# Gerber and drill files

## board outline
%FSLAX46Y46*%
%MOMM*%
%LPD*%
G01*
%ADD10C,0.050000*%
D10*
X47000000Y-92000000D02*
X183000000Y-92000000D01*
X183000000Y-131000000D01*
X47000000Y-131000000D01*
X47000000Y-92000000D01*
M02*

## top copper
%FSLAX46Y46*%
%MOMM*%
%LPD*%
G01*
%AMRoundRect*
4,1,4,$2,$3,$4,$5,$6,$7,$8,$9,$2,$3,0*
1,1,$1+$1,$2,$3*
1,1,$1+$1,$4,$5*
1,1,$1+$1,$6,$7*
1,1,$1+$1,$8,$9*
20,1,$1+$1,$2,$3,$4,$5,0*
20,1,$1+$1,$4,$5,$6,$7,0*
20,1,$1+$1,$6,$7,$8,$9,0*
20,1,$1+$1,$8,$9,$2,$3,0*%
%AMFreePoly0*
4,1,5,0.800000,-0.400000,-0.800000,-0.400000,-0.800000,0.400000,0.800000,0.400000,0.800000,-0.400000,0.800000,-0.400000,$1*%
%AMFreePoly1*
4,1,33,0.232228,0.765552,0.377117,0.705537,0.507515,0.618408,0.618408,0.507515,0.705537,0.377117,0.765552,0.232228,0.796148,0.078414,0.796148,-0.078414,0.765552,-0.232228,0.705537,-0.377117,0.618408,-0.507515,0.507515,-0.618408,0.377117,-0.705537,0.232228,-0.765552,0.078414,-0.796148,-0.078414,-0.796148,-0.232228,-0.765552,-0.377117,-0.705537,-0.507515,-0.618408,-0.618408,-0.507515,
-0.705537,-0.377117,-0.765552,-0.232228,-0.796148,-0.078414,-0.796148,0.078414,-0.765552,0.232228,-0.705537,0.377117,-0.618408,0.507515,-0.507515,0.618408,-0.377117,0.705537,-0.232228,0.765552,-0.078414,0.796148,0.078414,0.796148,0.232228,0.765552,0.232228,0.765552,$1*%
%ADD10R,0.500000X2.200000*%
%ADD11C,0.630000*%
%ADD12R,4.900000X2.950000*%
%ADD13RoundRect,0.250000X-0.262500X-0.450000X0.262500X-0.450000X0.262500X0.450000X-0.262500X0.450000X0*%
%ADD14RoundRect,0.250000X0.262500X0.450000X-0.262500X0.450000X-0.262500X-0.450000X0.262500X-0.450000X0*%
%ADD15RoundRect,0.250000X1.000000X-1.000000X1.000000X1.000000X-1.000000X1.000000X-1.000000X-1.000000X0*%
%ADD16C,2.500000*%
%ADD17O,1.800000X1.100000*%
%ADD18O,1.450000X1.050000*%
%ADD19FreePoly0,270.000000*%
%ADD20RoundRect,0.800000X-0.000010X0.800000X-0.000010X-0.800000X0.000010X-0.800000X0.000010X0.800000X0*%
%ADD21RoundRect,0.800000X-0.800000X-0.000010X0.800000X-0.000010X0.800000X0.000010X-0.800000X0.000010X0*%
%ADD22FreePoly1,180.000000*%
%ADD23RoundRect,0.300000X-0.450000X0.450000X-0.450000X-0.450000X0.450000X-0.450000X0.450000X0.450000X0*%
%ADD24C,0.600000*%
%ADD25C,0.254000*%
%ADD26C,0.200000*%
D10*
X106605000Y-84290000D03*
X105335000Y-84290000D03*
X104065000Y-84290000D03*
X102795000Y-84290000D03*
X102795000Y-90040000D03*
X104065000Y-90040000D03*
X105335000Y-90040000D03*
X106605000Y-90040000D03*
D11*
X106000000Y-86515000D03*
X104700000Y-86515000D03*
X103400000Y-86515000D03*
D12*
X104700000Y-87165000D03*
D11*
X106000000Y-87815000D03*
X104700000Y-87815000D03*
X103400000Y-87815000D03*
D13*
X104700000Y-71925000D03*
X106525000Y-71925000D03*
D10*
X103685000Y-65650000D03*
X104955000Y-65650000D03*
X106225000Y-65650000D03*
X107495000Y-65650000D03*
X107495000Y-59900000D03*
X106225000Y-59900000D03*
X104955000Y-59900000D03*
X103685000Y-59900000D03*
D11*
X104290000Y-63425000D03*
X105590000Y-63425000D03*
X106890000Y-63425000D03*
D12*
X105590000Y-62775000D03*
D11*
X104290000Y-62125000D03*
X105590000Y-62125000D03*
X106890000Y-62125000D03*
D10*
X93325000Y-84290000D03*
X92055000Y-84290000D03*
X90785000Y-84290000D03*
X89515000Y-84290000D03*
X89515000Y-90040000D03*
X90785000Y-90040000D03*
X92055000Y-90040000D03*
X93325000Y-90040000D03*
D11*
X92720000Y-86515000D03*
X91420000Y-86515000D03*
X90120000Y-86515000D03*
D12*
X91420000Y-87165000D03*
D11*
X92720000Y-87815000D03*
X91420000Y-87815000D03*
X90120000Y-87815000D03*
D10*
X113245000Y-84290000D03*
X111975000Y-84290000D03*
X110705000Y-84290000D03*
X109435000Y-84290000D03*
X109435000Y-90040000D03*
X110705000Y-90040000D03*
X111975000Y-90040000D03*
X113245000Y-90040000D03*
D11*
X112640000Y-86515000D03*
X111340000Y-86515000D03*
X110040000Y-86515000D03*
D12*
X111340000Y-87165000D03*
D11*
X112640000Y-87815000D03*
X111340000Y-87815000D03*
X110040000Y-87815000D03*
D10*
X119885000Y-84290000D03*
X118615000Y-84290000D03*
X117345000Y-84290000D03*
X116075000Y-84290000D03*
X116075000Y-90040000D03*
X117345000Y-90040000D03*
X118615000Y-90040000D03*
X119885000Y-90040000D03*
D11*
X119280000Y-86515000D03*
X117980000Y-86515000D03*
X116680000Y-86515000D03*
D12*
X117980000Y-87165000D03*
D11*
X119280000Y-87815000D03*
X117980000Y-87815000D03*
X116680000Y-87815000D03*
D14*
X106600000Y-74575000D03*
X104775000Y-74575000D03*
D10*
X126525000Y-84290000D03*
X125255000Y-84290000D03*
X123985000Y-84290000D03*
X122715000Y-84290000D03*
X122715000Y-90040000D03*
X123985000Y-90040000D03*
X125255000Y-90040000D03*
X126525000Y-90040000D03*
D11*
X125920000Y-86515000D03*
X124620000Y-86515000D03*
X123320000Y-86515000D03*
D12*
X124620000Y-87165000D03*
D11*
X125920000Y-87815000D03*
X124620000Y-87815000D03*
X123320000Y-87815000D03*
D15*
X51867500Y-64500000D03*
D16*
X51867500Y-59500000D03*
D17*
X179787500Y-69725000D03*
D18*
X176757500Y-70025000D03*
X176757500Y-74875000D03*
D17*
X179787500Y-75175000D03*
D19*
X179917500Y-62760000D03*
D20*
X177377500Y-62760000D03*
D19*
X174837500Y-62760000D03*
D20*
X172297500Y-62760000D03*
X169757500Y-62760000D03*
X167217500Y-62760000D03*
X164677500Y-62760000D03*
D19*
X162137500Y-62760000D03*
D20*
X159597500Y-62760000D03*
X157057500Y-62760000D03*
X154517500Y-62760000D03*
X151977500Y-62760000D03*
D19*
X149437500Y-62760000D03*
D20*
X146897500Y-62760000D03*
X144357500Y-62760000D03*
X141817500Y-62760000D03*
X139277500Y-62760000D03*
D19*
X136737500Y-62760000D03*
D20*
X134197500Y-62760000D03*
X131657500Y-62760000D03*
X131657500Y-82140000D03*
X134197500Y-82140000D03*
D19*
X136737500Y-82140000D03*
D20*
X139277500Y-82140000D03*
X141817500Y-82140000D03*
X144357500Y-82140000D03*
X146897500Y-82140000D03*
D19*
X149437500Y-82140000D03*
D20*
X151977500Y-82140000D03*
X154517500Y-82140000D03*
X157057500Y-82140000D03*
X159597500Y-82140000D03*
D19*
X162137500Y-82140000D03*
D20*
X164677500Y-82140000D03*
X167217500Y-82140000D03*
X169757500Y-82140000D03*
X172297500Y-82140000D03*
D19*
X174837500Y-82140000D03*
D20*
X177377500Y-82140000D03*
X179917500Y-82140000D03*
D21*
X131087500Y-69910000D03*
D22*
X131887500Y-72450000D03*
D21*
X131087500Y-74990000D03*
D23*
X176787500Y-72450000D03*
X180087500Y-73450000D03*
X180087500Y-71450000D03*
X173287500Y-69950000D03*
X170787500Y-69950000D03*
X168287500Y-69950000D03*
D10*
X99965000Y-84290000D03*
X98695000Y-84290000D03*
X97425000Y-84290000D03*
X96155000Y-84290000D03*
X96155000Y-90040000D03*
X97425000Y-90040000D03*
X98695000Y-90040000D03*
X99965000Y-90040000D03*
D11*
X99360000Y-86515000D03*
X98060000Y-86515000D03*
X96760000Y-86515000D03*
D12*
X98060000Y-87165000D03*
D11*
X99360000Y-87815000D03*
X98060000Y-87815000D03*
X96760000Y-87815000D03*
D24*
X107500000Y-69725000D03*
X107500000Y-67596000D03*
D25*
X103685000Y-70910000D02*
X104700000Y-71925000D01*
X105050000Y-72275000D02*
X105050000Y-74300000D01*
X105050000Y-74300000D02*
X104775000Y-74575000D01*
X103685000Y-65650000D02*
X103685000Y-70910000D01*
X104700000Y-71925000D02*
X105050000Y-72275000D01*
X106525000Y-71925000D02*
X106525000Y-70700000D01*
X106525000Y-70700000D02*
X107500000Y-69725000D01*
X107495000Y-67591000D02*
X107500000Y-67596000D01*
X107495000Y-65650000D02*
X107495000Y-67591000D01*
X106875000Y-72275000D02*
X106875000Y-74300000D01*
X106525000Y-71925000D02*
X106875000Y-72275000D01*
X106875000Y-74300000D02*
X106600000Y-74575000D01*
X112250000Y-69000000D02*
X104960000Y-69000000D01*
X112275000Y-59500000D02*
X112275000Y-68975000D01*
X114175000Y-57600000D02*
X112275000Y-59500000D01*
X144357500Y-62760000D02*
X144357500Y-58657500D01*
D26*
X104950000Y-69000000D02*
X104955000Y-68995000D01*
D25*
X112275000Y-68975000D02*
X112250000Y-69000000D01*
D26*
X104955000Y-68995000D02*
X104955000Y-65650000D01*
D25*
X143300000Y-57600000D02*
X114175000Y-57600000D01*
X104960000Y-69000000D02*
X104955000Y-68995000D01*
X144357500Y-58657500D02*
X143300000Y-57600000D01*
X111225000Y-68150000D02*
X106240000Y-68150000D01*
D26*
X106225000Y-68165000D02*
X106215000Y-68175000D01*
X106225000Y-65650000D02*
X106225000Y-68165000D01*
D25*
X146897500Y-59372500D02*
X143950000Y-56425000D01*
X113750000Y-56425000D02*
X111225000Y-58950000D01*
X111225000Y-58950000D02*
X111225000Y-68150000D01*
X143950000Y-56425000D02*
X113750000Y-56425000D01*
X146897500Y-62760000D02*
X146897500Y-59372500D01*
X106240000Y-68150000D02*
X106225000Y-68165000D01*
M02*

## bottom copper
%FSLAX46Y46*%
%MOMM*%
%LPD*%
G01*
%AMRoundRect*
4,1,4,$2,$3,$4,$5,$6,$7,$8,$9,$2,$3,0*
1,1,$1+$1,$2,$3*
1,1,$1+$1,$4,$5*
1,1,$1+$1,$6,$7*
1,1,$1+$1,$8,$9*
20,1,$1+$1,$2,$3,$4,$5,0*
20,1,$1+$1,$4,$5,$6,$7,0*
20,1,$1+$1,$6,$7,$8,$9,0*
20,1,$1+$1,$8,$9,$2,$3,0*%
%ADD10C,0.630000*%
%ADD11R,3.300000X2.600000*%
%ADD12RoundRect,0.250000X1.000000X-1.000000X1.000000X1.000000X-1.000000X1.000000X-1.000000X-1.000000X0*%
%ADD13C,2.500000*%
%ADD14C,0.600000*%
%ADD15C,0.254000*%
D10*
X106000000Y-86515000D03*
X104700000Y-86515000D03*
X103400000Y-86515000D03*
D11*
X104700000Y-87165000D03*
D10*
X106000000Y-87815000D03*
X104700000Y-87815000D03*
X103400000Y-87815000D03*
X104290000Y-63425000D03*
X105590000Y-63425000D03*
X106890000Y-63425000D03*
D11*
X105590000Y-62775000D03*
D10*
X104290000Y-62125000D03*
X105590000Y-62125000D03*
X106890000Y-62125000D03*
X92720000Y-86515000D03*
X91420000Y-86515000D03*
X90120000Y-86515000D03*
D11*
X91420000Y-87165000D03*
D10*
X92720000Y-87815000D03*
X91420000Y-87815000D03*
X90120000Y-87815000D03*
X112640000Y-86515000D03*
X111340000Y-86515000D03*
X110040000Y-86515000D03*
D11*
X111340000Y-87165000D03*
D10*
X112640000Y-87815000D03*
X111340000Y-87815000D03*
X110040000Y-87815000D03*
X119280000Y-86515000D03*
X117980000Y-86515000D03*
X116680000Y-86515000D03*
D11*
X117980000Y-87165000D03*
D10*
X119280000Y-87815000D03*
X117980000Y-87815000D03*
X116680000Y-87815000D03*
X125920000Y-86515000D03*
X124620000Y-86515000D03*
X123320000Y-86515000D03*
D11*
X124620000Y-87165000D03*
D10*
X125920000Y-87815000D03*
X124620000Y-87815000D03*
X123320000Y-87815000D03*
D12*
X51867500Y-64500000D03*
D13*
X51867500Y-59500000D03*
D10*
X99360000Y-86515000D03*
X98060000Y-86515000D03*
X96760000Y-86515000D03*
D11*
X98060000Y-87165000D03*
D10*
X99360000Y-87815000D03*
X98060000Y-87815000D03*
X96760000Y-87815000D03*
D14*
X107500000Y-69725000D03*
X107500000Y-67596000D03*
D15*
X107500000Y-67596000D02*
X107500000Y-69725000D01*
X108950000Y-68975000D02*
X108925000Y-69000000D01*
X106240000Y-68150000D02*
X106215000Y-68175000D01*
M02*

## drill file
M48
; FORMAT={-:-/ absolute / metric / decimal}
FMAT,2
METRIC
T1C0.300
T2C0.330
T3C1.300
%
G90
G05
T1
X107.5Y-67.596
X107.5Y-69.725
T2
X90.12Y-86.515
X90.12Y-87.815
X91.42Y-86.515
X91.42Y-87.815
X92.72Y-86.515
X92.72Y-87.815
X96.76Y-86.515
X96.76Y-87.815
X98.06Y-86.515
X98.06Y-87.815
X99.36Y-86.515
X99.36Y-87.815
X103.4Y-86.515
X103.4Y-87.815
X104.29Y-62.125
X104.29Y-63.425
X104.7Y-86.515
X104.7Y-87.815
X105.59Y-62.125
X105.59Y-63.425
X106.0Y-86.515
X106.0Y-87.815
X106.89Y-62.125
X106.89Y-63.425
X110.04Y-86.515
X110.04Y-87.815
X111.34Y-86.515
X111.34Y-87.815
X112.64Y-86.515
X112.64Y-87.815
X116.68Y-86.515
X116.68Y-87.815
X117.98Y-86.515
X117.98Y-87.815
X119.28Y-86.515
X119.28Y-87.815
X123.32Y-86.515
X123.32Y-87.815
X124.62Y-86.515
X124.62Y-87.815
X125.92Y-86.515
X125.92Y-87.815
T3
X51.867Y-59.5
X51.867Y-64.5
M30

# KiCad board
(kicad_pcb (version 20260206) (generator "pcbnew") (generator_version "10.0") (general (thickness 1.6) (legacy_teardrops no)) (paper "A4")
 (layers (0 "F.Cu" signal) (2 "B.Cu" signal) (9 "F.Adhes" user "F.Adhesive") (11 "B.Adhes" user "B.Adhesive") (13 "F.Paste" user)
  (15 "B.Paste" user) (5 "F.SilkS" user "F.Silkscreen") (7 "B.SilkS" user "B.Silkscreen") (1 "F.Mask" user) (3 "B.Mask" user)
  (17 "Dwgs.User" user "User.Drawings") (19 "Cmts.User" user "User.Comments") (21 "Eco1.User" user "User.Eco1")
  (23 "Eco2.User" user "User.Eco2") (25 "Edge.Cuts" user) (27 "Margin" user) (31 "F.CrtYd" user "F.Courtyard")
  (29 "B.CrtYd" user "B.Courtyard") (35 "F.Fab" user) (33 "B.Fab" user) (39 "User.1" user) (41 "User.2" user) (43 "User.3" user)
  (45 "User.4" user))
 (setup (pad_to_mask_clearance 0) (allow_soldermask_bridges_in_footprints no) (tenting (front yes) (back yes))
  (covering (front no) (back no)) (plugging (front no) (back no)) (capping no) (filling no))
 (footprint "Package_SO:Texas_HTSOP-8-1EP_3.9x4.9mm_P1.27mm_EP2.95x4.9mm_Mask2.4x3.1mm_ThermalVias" (layer "F.Cu") (at 104.7 87.165 -90)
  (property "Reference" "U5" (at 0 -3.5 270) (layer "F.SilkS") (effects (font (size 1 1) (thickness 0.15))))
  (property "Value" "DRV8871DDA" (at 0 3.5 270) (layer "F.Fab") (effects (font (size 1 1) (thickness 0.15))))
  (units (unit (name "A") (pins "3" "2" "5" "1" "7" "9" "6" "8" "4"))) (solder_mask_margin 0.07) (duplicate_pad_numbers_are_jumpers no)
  (pad "" smd rect (at 0 0 270) (size 2.4 3.1) (layers "F.Mask"))
  (pad "" smd rect (at 0 0 270) (size 2.4 3.1) (layers "F.Paste"))
  (pad "1" smd rect (at -2.875 -1.905 270) (size 2.2 0.5) (layers "F.Cu" "F.Mask" "F.Paste") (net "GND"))
  (pad "2" smd rect (at -2.875 -0.635 270) (size 2.2 0.5) (layers "F.Cu" "F.Mask" "F.Paste") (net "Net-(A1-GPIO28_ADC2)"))
  (pad "3" smd rect (at -2.875 0.635 270) (size 2.2 0.5) (layers "F.Cu" "F.Mask" "F.Paste") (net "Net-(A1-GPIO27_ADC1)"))
  (pad "4" smd rect (at -2.875 1.905 270) (size 2.2 0.5) (layers "F.Cu" "F.Mask" "F.Paste") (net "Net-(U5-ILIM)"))
  (pad "5" smd rect (at 2.875 1.905 270) (size 2.2 0.5) (layers "F.Cu" "F.Mask" "F.Paste") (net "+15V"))
  (pad "6" smd rect (at 2.875 0.635 270) (size 2.2 0.5) (layers "F.Cu" "F.Mask" "F.Paste") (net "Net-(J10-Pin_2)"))
  (pad "7" smd rect (at 2.875 -0.635 270) (size 2.2 0.5) (layers "F.Cu" "F.Mask" "F.Paste") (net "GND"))
  (pad "8" smd rect (at 2.875 -1.905 270) (size 2.2 0.5) (layers "F.Cu" "F.Mask" "F.Paste") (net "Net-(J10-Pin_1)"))
  (pad "9" thru_hole circle (at -0.65 -1.3 270) (size 0.63 0.63) (drill 0.33) (layers "*.Cu" "*.Mask") (remove_unused_layers no) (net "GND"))
  (pad "9" thru_hole circle (at -0.65 0 270) (size 0.63 0.63) (drill 0.33) (layers "*.Cu" "*.Mask") (remove_unused_layers no) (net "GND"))
  (pad "9" thru_hole circle (at -0.65 1.3 270) (size 0.63 0.63) (drill 0.33) (layers "*.Cu" "*.Mask") (remove_unused_layers no) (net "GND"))
  (pad "9" smd rect (at 0 0 270) (size 2.6 3.3) (layers "B.Cu") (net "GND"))
  (pad "9" smd rect (at 0 0 270) (size 2.95 4.9) (layers "F.Cu") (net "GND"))
  (pad "9" thru_hole circle (at 0.65 -1.3 270) (size 0.63 0.63) (drill 0.33) (layers "*.Cu" "*.Mask") (remove_unused_layers no) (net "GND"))
  (pad "9" thru_hole circle (at 0.65 0 270) (size 0.63 0.63) (drill 0.33) (layers "*.Cu" "*.Mask") (remove_unused_layers no) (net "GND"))
  (pad "9" thru_hole circle (at 0.65 1.3 270) (size 0.63 0.63) (drill 0.33) (layers "*.Cu" "*.Mask") (remove_unused_layers no) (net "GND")))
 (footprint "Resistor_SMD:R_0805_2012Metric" (layer "F.Cu") (at 105.6125 71.925)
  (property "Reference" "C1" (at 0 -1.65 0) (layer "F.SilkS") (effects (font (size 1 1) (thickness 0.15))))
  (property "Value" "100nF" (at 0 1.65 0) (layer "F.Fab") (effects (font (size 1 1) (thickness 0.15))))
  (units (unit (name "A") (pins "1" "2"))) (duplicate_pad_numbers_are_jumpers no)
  (pad "1" smd roundrect (at -0.9125 0) (size 1.025 1.4) (layers "F.Cu" "F.Mask" "F.Paste") (roundrect_rratio 0.243902) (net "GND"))
  (pad "2" smd roundrect (at 0.9125 0) (size 1.025 1.4) (layers "F.Cu" "F.Mask" "F.Paste") (roundrect_rratio 0.243902) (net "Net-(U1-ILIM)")))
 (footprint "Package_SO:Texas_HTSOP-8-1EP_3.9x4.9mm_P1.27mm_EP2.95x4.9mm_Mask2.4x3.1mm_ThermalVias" (layer "F.Cu") (at 105.59 62.775 90)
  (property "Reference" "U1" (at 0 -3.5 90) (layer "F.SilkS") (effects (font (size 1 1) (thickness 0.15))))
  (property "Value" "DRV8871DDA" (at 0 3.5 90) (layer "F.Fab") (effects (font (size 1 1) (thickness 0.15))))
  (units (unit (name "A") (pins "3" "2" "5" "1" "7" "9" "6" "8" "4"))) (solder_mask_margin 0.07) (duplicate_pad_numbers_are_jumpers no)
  (pad "" smd rect (at 0 0 90) (size 2.4 3.1) (layers "F.Mask"))
  (pad "" smd rect (at 0 0 90) (size 2.4 3.1) (layers "F.Paste"))
  (pad "1" smd rect (at -2.875 -1.905 90) (size 2.2 0.5) (layers "F.Cu" "F.Mask" "F.Paste") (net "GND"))
  (pad "2" smd rect (at -2.875 -0.635 90) (size 2.2 0.5) (layers "F.Cu" "F.Mask" "F.Paste") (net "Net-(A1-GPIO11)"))
  (pad "3" smd rect (at -2.875 0.635 90) (size 2.2 0.5) (layers "F.Cu" "F.Mask" "F.Paste") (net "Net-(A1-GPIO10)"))
  (pad "4" smd rect (at -2.875 1.905 90) (size 2.2 0.5) (layers "F.Cu" "F.Mask" "F.Paste") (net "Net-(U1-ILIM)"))
  (pad "5" smd rect (at 2.875 1.905 90) (size 2.2 0.5) (layers "F.Cu" "F.Mask" "F.Paste") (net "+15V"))
  (pad "6" smd rect (at 2.875 0.635 90) (size 2.2 0.5) (layers "F.Cu" "F.Mask" "F.Paste") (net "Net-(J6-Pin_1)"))
  (pad "7" smd rect (at 2.875 -0.635 90) (size 2.2 0.5) (layers "F.Cu" "F.Mask" "F.Paste") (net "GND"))
  (pad "8" smd rect (at 2.875 -1.905 90) (size 2.2 0.5) (layers "F.Cu" "F.Mask" "F.Paste") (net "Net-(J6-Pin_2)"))
  (pad "9" thru_hole circle (at -0.65 -1.3 90) (size 0.63 0.63) (drill 0.33) (layers "*.Cu" "*.Mask") (remove_unused_layers no) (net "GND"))
  (pad "9" thru_hole circle (at -0.65 0 90) (size 0.63 0.63) (drill 0.33) (layers "*.Cu" "*.Mask") (remove_unused_layers no) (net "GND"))
  (pad "9" thru_hole circle (at -0.65 1.3 90) (size 0.63 0.63) (drill 0.33) (layers "*.Cu" "*.Mask") (remove_unused_layers no) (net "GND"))
  (pad "9" smd rect (at 0 0 90) (size 2.6 3.3) (layers "B.Cu") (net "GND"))
  (pad "9" smd rect (at 0 0 90) (size 2.95 4.9) (layers "F.Cu") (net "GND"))
  (pad "9" thru_hole circle (at 0.65 -1.3 90) (size 0.63 0.63) (drill 0.33) (layers "*.Cu" "*.Mask") (remove_unused_layers no) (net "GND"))
  (pad "9" thru_hole circle (at 0.65 0 90) (size 0.63 0.63) (drill 0.33) (layers "*.Cu" "*.Mask") (remove_unused_layers no) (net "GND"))
  (pad "9" thru_hole circle (at 0.65 1.3 90) (size 0.63 0.63) (drill 0.33) (layers "*.Cu" "*.Mask") (remove_unused_layers no) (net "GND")))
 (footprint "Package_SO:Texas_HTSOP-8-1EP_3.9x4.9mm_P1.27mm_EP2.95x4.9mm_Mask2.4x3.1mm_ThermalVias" (layer "F.Cu") (at 91.42 87.165 -90)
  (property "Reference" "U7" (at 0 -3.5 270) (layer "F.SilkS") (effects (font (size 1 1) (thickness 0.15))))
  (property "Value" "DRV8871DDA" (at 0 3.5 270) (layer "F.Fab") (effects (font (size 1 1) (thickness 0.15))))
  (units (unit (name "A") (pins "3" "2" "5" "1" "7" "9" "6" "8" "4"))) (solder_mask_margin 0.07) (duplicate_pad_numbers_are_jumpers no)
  (pad "" smd rect (at 0 0 270) (size 2.4 3.1) (layers "F.Mask"))
  (pad "" smd rect (at 0 0 270) (size 2.4 3.1) (layers "F.Paste"))
  (pad "1" smd rect (at -2.875 -1.905 270) (size 2.2 0.5) (layers "F.Cu" "F.Mask" "F.Paste") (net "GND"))
  (pad "2" smd rect (at -2.875 -0.635 270) (size 2.2 0.5) (layers "F.Cu" "F.Mask" "F.Paste") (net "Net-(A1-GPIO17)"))
  (pad "3" smd rect (at -2.875 0.635 270) (size 2.2 0.5) (layers "F.Cu" "F.Mask" "F.Paste") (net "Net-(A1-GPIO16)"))
  (pad "4" smd rect (at -2.875 1.905 270) (size 2.2 0.5) (layers "F.Cu" "F.Mask" "F.Paste") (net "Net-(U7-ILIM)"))
  (pad "5" smd rect (at 2.875 1.905 270) (size 2.2 0.5) (layers "F.Cu" "F.Mask" "F.Paste") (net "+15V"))
  (pad "6" smd rect (at 2.875 0.635 270) (size 2.2 0.5) (layers "F.Cu" "F.Mask" "F.Paste") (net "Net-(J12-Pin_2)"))
  (pad "7" smd rect (at 2.875 -0.635 270) (size 2.2 0.5) (layers "F.Cu" "F.Mask" "F.Paste") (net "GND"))
  (pad "8" smd rect (at 2.875 -1.905 270) (size 2.2 0.5) (layers "F.Cu" "F.Mask" "F.Paste") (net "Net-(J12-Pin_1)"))
  (pad "9" thru_hole circle (at -0.65 -1.3 270) (size 0.63 0.63) (drill 0.33) (layers "*.Cu" "*.Mask") (remove_unused_layers no) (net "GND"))
  (pad "9" thru_hole circle (at -0.65 0 270) (size 0.63 0.63) (drill 0.33) (layers "*.Cu" "*.Mask") (remove_unused_layers no) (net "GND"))
  (pad "9" thru_hole circle (at -0.65 1.3 270) (size 0.63 0.63) (drill 0.33) (layers "*.Cu" "*.Mask") (remove_unused_layers no) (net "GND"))
  (pad "9" smd rect (at 0 0 270) (size 2.6 3.3) (layers "B.Cu") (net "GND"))
  (pad "9" smd rect (at 0 0 270) (size 2.95 4.9) (layers "F.Cu") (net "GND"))
  (pad "9" thru_hole circle (at 0.65 -1.3 270) (size 0.63 0.63) (drill 0.33) (layers "*.Cu" "*.Mask") (remove_unused_layers no) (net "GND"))
  (pad "9" thru_hole circle (at 0.65 0 270) (size 0.63 0.63) (drill 0.33) (layers "*.Cu" "*.Mask") (remove_unused_layers no) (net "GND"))
  (pad "9" thru_hole circle (at 0.65 1.3 270) (size 0.63 0.63) (drill 0.33) (layers "*.Cu" "*.Mask") (remove_unused_layers no) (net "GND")))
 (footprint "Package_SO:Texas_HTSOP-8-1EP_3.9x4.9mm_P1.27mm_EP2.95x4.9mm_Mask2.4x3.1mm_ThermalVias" (layer "F.Cu") (at 111.34 87.165 -90)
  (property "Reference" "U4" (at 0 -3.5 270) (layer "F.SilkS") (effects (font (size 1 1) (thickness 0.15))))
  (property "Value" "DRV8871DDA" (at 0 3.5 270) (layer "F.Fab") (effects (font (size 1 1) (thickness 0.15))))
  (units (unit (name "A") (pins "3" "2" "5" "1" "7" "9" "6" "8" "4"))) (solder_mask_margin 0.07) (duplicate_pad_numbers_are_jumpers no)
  (pad "" smd rect (at 0 0 270) (size 2.4 3.1) (layers "F.Mask"))
  (pad "" smd rect (at 0 0 270) (size 2.4 3.1) (layers "F.Paste"))
  (pad "1" smd rect (at -2.875 -1.905 270) (size 2.2 0.5) (layers "F.Cu" "F.Mask" "F.Paste") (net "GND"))
  (pad "2" smd rect (at -2.875 -0.635 270) (size 2.2 0.5) (layers "F.Cu" "F.Mask" "F.Paste") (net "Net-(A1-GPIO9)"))
  (pad "3" smd rect (at -2.875 0.635 270) (size 2.2 0.5) (layers "F.Cu" "F.Mask" "F.Paste") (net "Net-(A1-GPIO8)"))
  (pad "4" smd rect (at -2.875 1.905 270) (size 2.2 0.5) (layers "F.Cu" "F.Mask" "F.Paste") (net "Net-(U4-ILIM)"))
  (pad "5" smd rect (at 2.875 1.905 270) (size 2.2 0.5) (layers "F.Cu" "F.Mask" "F.Paste") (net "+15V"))
  (pad "6" smd rect (at 2.875 0.635 270) (size 2.2 0.5) (layers "F.Cu" "F.Mask" "F.Paste") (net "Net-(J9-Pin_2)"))
  (pad "7" smd rect (at 2.875 -0.635 270) (size 2.2 0.5) (layers "F.Cu" "F.Mask" "F.Paste") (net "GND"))
  (pad "8" smd rect (at 2.875 -1.905 270) (size 2.2 0.5) (layers "F.Cu" "F.Mask" "F.Paste") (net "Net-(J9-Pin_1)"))
  (pad "9" thru_hole circle (at -0.65 -1.3 270) (size 0.63 0.63) (drill 0.33) (layers "*.Cu" "*.Mask") (remove_unused_layers no) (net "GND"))
  (pad "9" thru_hole circle (at -0.65 0 270) (size 0.63 0.63) (drill 0.33) (layers "*.Cu" "*.Mask") (remove_unused_layers no) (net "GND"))
  (pad "9" thru_hole circle (at -0.65 1.3 270) (size 0.63 0.63) (drill 0.33) (layers "*.Cu" "*.Mask") (remove_unused_layers no) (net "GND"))
  (pad "9" smd rect (at 0 0 270) (size 2.6 3.3) (layers "B.Cu") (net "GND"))
  (pad "9" smd rect (at 0 0 270) (size 2.95 4.9) (layers "F.Cu") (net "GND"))
  (pad "9" thru_hole circle (at 0.65 -1.3 270) (size 0.63 0.63) (drill 0.33) (layers "*.Cu" "*.Mask") (remove_unused_layers no) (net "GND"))
  (pad "9" thru_hole circle (at 0.65 0 270) (size 0.63 0.63) (drill 0.33) (layers "*.Cu" "*.Mask") (remove_unused_layers no) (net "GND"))
  (pad "9" thru_hole circle (at 0.65 1.3 270) (size 0.63 0.63) (drill 0.33) (layers "*.Cu" "*.Mask") (remove_unused_layers no) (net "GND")))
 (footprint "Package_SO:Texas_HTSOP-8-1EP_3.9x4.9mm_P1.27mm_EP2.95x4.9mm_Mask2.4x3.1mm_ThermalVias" (layer "F.Cu") (at 117.98 87.165 -90)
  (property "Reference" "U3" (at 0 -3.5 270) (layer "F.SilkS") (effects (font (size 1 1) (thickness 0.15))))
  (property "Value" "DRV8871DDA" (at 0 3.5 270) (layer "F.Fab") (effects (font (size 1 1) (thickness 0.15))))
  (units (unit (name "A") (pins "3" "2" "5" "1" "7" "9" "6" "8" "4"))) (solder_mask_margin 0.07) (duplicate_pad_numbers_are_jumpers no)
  (pad "" smd rect (at 0 0 270) (size 2.4 3.1) (layers "F.Mask"))
  (pad "" smd rect (at 0 0 270) (size 2.4 3.1) (layers "F.Paste"))
  (pad "1" smd rect (at -2.875 -1.905 270) (size 2.2 0.5) (layers "F.Cu" "F.Mask" "F.Paste") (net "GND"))
  (pad "2" smd rect (at -2.875 -0.635 270) (size 2.2 0.5) (layers "F.Cu" "F.Mask" "F.Paste") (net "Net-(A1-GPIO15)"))
  (pad "3" smd rect (at -2.875 0.635 270) (size 2.2 0.5) (layers "F.Cu" "F.Mask" "F.Paste") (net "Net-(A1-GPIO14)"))
  (pad "4" smd rect (at -2.875 1.905 270) (size 2.2 0.5) (layers "F.Cu" "F.Mask" "F.Paste") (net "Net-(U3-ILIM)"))
  (pad "5" smd rect (at 2.875 1.905 270) (size 2.2 0.5) (layers "F.Cu" "F.Mask" "F.Paste") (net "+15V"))
  (pad "6" smd rect (at 2.875 0.635 270) (size 2.2 0.5) (layers "F.Cu" "F.Mask" "F.Paste") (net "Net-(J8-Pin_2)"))
  (pad "7" smd rect (at 2.875 -0.635 270) (size 2.2 0.5) (layers "F.Cu" "F.Mask" "F.Paste") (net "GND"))
  (pad "8" smd rect (at 2.875 -1.905 270) (size 2.2 0.5) (layers "F.Cu" "F.Mask" "F.Paste") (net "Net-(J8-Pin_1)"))
  (pad "9" thru_hole circle (at -0.65 -1.3 270) (size 0.63 0.63) (drill 0.33) (layers "*.Cu" "*.Mask") (remove_unused_layers no) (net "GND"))
  (pad "9" thru_hole circle (at -0.65 0 270) (size 0.63 0.63) (drill 0.33) (layers "*.Cu" "*.Mask") (remove_unused_layers no) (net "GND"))
  (pad "9" thru_hole circle (at -0.65 1.3 270) (size 0.63 0.63) (drill 0.33) (layers "*.Cu" "*.Mask") (remove_unused_layers no) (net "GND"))
  (pad "9" smd rect (at 0 0 270) (size 2.6 3.3) (layers "B.Cu") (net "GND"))
  (pad "9" smd rect (at 0 0 270) (size 2.95 4.9) (layers "F.Cu") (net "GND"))
  (pad "9" thru_hole circle (at 0.65 -1.3 270) (size 0.63 0.63) (drill 0.33) (layers "*.Cu" "*.Mask") (remove_unused_layers no) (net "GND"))
  (pad "9" thru_hole circle (at 0.65 0 270) (size 0.63 0.63) (drill 0.33) (layers "*.Cu" "*.Mask") (remove_unused_layers no) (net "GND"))
  (pad "9" thru_hole circle (at 0.65 1.3 270) (size 0.63 0.63) (drill 0.33) (layers "*.Cu" "*.Mask") (remove_unused_layers no) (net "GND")))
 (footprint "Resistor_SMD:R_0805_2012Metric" (layer "F.Cu") (at 105.6875 74.575 180)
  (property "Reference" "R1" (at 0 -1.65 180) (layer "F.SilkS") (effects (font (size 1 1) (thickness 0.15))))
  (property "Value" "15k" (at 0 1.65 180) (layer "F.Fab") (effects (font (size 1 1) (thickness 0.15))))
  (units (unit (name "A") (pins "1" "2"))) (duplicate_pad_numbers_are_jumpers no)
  (pad "1" smd roundrect (at -0.9125 0 180) (size 1.025 1.4) (layers "F.Cu" "F.Mask" "F.Paste") (roundrect_rratio 0.243902)
   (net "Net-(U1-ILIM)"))
  (pad "2" smd roundrect (at 0.9125 0 180) (size 1.025 1.4) (layers "F.Cu" "F.Mask" "F.Paste") (roundrect_rratio 0.243902) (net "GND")))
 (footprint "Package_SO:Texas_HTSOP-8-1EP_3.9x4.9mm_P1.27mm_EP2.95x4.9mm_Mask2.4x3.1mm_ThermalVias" (layer "F.Cu") (at 124.62 87.165 -90)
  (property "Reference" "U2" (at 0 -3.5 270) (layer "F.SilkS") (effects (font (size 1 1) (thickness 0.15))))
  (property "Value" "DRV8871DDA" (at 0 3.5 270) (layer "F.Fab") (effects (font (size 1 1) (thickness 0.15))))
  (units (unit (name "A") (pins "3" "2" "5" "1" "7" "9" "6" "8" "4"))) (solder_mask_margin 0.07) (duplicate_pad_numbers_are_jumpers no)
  (pad "" smd rect (at 0 0 270) (size 2.4 3.1) (layers "F.Mask"))
  (pad "" smd rect (at 0 0 270) (size 2.4 3.1) (layers "F.Paste"))
  (pad "1" smd rect (at -2.875 -1.905 270) (size 2.2 0.5) (layers "F.Cu" "F.Mask" "F.Paste") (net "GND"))
  (pad "2" smd rect (at -2.875 -0.635 270) (size 2.2 0.5) (layers "F.Cu" "F.Mask" "F.Paste") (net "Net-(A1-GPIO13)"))
  (pad "3" smd rect (at -2.875 0.635 270) (size 2.2 0.5) (layers "F.Cu" "F.Mask" "F.Paste") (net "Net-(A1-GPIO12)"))
  (pad "4" smd rect (at -2.875 1.905 270) (size 2.2 0.5) (layers "F.Cu" "F.Mask" "F.Paste") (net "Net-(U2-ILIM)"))
  (pad "5" smd rect (at 2.875 1.905 270) (size 2.2 0.5) (layers "F.Cu" "F.Mask" "F.Paste") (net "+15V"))
  (pad "6" smd rect (at 2.875 0.635 270) (size 2.2 0.5) (layers "F.Cu" "F.Mask" "F.Paste") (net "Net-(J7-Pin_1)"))
  (pad "7" smd rect (at 2.875 -0.635 270) (size 2.2 0.5) (layers "F.Cu" "F.Mask" "F.Paste") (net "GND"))
  (pad "8" smd rect (at 2.875 -1.905 270) (size 2.2 0.5) (layers "F.Cu" "F.Mask" "F.Paste") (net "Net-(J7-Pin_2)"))
  (pad "9" thru_hole circle (at -0.65 -1.3 270) (size 0.63 0.63) (drill 0.33) (layers "*.Cu" "*.Mask") (remove_unused_layers no) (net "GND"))
  (pad "9" thru_hole circle (at -0.65 0 270) (size 0.63 0.63) (drill 0.33) (layers "*.Cu" "*.Mask") (remove_unused_layers no) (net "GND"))
  (pad "9" thru_hole circle (at -0.65 1.3 270) (size 0.63 0.63) (drill 0.33) (layers "*.Cu" "*.Mask") (remove_unused_layers no) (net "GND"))
  (pad "9" smd rect (at 0 0 270) (size 2.6 3.3) (layers "B.Cu") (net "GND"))
  (pad "9" smd rect (at 0 0 270) (size 2.95 4.9) (layers "F.Cu") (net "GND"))
  (pad "9" thru_hole circle (at 0.65 -1.3 270) (size 0.63 0.63) (drill 0.33) (layers "*.Cu" "*.Mask") (remove_unused_layers no) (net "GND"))
  (pad "9" thru_hole circle (at 0.65 0 270) (size 0.63 0.63) (drill 0.33) (layers "*.Cu" "*.Mask") (remove_unused_layers no) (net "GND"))
  (pad "9" thru_hole circle (at 0.65 1.3 270) (size 0.63 0.63) (drill 0.33) (layers "*.Cu" "*.Mask") (remove_unused_layers no) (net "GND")))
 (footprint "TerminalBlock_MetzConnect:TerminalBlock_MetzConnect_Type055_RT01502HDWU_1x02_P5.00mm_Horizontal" (layer "F.Cu")
  (at 51.8675 64.5 90)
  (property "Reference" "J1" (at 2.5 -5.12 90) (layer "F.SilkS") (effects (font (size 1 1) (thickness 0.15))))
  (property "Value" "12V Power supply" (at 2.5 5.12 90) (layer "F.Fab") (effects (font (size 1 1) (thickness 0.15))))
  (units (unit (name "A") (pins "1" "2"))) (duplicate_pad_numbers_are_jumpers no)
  (pad "1" thru_hole roundrect (at 0 0 90) (size 2.5 2.5) (drill 1.3) (layers "*.Cu" "*.Mask") (remove_unused_layers no)
   (roundrect_rratio 0.1) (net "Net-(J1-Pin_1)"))
  (pad "2" thru_hole circle (at 5 0 90) (size 2.5 2.5) (drill 1.3) (layers "*.Cu" "*.Mask") (remove_unused_layers no) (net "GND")))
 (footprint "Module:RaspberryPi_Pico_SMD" (layer "F.Cu") (at 155.7875 72.45 -90)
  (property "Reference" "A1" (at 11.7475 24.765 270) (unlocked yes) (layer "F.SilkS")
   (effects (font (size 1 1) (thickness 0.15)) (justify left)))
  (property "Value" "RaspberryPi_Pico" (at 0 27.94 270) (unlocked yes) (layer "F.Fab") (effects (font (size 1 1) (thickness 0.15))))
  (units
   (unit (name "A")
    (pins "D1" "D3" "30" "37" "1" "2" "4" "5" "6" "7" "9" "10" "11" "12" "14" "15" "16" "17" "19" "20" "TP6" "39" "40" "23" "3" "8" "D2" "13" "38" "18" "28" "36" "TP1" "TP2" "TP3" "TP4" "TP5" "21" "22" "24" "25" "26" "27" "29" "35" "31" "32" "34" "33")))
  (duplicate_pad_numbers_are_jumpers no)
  (pad "" smd rect (at -8.89 -24.13 270) (size 3.8 2.2) (drill (offset -0.8 0)) (layers "F.Paste"))
  (pad "" smd rect (at -8.89 -21.59 270) (size 3.8 2.2) (drill (offset -0.8 0)) (layers "F.Paste"))
  (pad "" smd rect (at -8.89 -19.05 270) (size 3.8 2.2) (drill (offset -0.8 0)) (layers "F.Paste"))
  (pad "" smd rect (at -8.89 -16.51 270) (size 3.8 2.2) (drill (offset -0.8 0)) (layers "F.Paste"))
  (pad "" smd rect (at -8.89 -13.97 270) (size 3.8 2.2) (drill (offset -0.8 0)) (layers "F.Paste"))
  (pad "" smd rect (at -8.89 -11.43 270) (size 3.8 2.2) (drill (offset -0.8 0)) (layers "F.Paste"))
  (pad "" smd rect (at -8.89 -8.89 270) (size 3.8 2.2) (drill (offset -0.8 0)) (layers "F.Paste"))
  (pad "" smd rect (at -8.89 -6.35 270) (size 3.8 2.2) (drill (offset -0.8 0)) (layers "F.Paste"))
  (pad "" smd rect (at -8.89 -3.81 270) (size 3.8 2.2) (drill (offset -0.8 0)) (layers "F.Paste"))
  (pad "" smd rect (at -8.89 -1.27 270) (size 3.8 2.2) (drill (offset -0.8 0)) (layers "F.Paste"))
  (pad "" smd rect (at -8.89 1.27 270) (size 3.8 2.2) (drill (offset -0.8 0)) (layers "F.Paste"))
  (pad "" smd rect (at -8.89 3.81 270) (size 3.8 2.2) (drill (offset -0.8 0)) (layers "F.Paste"))
  (pad "" smd rect (at -8.89 6.35 270) (size 3.8 2.2) (drill (offset -0.8 0)) (layers "F.Paste"))
  (pad "" smd rect (at -8.89 8.89 270) (size 3.8 2.2) (drill (offset -0.8 0)) (layers "F.Paste"))
  (pad "" smd rect (at -8.89 11.43 270) (size 3.8 2.2) (drill (offset -0.8 0)) (layers "F.Paste"))
  (pad "" smd rect (at -8.89 13.97 270) (size 3.8 2.2) (drill (offset -0.8 0)) (layers "F.Paste"))
  (pad "" smd rect (at -8.89 16.51 270) (size 3.8 2.2) (drill (offset -0.8 0)) (layers "F.Paste"))
  (pad "" smd rect (at -8.89 19.05 270) (size 3.8 2.2) (drill (offset -0.8 0)) (layers "F.Paste"))
  (pad "" smd rect (at -8.89 21.59 270) (size 3.8 2.2) (drill (offset -0.8 0)) (layers "F.Paste"))
  (pad "" smd rect (at -8.89 24.13 270) (size 3.8 2.2) (drill (offset -0.8 0)) (layers "F.Paste"))
  (pad "" smd oval (at -2.725 -24 270) (size 1.1 1.8) (layers "F.Cu" "F.Mask" "F.Paste"))
  (pad "" smd rect (at -2.54 23.9 270) (size 2.2 3.8) (drill (offset 0 0.8)) (layers "F.Paste"))
  (pad "" smd oval (at -2.425 -20.97 270) (size 1.05 1.45) (layers "F.Cu" "F.Mask" "F.Paste"))
  (pad "" smd rect (at 0 23.9 270) (size 2.2 3.8) (drill (offset 0 0.8)) (layers "F.Paste"))
  (pad "" smd oval (at 2.425 -20.97 270) (size 1.05 1.45) (layers "F.Cu" "F.Mask" "F.Paste"))
  (pad "" smd rect (at 2.54 23.9 270) (size 2.2 3.8) (drill (offset 0 0.8)) (layers "F.Paste"))
  (pad "" smd oval (at 2.725 -24 270) (size 1.1 1.8) (layers "F.Cu" "F.Mask" "F.Paste"))
  (pad "" smd rect (at 8.89 -24.13 270) (size 3.8 2.2) (drill (offset 0.8 0)) (layers "F.Paste"))
  (pad "" smd rect (at 8.89 -21.59 270) (size 3.8 2.2) (drill (offset 0.8 0)) (layers "F.Paste"))
  (pad "" smd rect (at 8.89 -19.05 270) (size 3.8 2.2) (drill (offset 0.8 0)) (layers "F.Paste"))
  (pad "" smd rect (at 8.89 -16.51 270) (size 3.8 2.2) (drill (offset 0.8 0)) (layers "F.Paste"))
  (pad "" smd rect (at 8.89 -13.97 270) (size 3.8 2.2) (drill (offset 0.8 0)) (layers "F.Paste"))
  (pad "" smd rect (at 8.89 -11.43 270) (size 3.8 2.2) (drill (offset 0.8 0)) (layers "F.Paste"))
  (pad "" smd rect (at 8.89 -8.89 270) (size 3.8 2.2) (drill (offset 0.8 0)) (layers "F.Paste"))
  (pad "" smd rect (at 8.89 -6.35 270) (size 3.8 2.2) (drill (offset 0.8 0)) (layers "F.Paste"))
  (pad "" smd rect (at 8.89 -3.81 270) (size 3.8 2.2) (drill (offset 0.8 0)) (layers "F.Paste"))
  (pad "" smd rect (at 8.89 -1.27 270) (size 3.8 2.2) (drill (offset 0.8 0)) (layers "F.Paste"))
  (pad "" smd rect (at 8.89 1.27 270) (size 3.8 2.2) (drill (offset 0.8 0)) (layers "F.Paste"))
  (pad "" smd rect (at 8.89 3.81 270) (size 3.8 2.2) (drill (offset 0.8 0)) (layers "F.Paste"))
  (pad "" smd rect (at 8.89 6.35 270) (size 3.8 2.2) (drill (offset 0.8 0)) (layers "F.Paste"))
  (pad "" smd rect (at 8.89 8.89 270) (size 3.8 2.2) (drill (offset 0.8 0)) (layers "F.Paste"))
  (pad "" smd rect (at 8.89 11.43 270) (size 3.8 2.2) (drill (offset 0.8 0)) (layers "F.Paste"))
  (pad "" smd rect (at 8.89 13.97 270) (size 3.8 2.2) (drill (offset 0.8 0)) (layers "F.Paste"))
  (pad "" smd rect (at 8.89 16.51 270) (size 3.8 2.2) (drill (offset 0.8 0)) (layers "F.Paste"))
  (pad "" smd rect (at 8.89 19.05 270) (size 3.8 2.2) (drill (offset 0.8 0)) (layers "F.Paste"))
  (pad "" smd rect (at 8.89 21.59 270) (size 3.8 2.2) (drill (offset 0.8 0)) (layers "F.Paste"))
  (pad "" smd rect (at 8.89 24.13 270) (size 3.8 2.2) (drill (offset 0.8 0)) (layers "F.Paste"))
  (pad "1" smd custom (at -9.69 -24.13 270) (size 1.6 0.8) (layers "F.Cu" "F.Mask") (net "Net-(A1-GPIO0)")
   (options (clearance outline) (anchor rect)) (primitives))
  (pad "2" smd roundrect (at -9.69 -21.59 270) (size 3.2 1.6) (layers "F.Cu" "F.Mask") (roundrect_rratio 0.5) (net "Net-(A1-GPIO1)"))
  (pad "3" smd custom (at -9.69 -19.05 270) (size 1.6 0.8) (layers "F.Cu" "F.Mask") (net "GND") (options (clearance outline) (anchor rect))
   (primitives))
  (pad "4" smd roundrect (at -9.69 -16.51 270) (size 3.2 1.6) (layers "F.Cu" "F.Mask") (roundrect_rratio 0.5)
   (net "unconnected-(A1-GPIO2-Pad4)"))
  (pad "5" smd roundrect (at -9.69 -13.97 270) (size 3.2 1.6) (layers "F.Cu" "F.Mask") (roundrect_rratio 0.5)
   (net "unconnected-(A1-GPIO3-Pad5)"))
  (pad "6" smd roundrect (at -9.69 -11.43 270) (size 3.2 1.6) (layers "F.Cu" "F.Mask") (roundrect_rratio 0.5) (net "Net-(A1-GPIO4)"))
  (pad "7" smd roundrect (at -9.69 -8.89 270) (size 3.2 1.6) (layers "F.Cu" "F.Mask") (roundrect_rratio 0.5) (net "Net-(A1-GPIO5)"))
  (pad "8" smd custom (at -9.69 -6.35 270) (size 1.6 0.8) (layers "F.Cu" "F.Mask") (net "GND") (options (clearance outline) (anchor rect))
   (primitives))
  (pad "9" smd roundrect (at -9.69 -3.81 270) (size 3.2 1.6) (layers "F.Cu" "F.Mask") (roundrect_rratio 0.5) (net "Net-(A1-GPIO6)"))
  (pad "10" smd roundrect (at -9.69 -1.27 270) (size 3.2 1.6) (layers "F.Cu" "F.Mask") (roundrect_rratio 0.5) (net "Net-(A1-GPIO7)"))
  (pad "11" smd roundrect (at -9.69 1.27 270) (size 3.2 1.6) (layers "F.Cu" "F.Mask") (roundrect_rratio 0.5) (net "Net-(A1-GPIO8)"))
  (pad "12" smd roundrect (at -9.69 3.81 270) (size 3.2 1.6) (layers "F.Cu" "F.Mask") (roundrect_rratio 0.5) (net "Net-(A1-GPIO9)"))
  (pad "13" smd custom (at -9.69 6.35 270) (size 1.6 0.8) (layers "F.Cu" "F.Mask") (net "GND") (options (clearance outline) (anchor rect))
   (primitives))
  (pad "14" smd roundrect (at -9.69 8.89 270) (size 3.2 1.6) (layers "F.Cu" "F.Mask") (roundrect_rratio 0.5) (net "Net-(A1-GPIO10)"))
  (pad "15" smd roundrect (at -9.69 11.43 270) (size 3.2 1.6) (layers "F.Cu" "F.Mask") (roundrect_rratio 0.5) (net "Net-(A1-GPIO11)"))
  (pad "16" smd roundrect (at -9.69 13.97 270) (size 3.2 1.6) (layers "F.Cu" "F.Mask") (roundrect_rratio 0.5) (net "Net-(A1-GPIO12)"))
  (pad "17" smd roundrect (at -9.69 16.51 270) (size 3.2 1.6) (layers "F.Cu" "F.Mask") (roundrect_rratio 0.5) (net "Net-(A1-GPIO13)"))
  (pad "18" smd custom (at -9.69 19.05 270) (size 1.6 0.8) (layers "F.Cu" "F.Mask") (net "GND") (options (clearance outline) (anchor rect))
   (primitives))
  (pad "19" smd roundrect (at -9.69 21.59 270) (size 3.2 1.6) (layers "F.Cu" "F.Mask") (roundrect_rratio 0.5) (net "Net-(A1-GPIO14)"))
  (pad "20" smd roundrect (at -9.69 24.13 270) (size 3.2 1.6) (layers "F.Cu" "F.Mask") (roundrect_rratio 0.5) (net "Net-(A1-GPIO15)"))
  (pad "21" smd roundrect (at 9.69 24.13 270) (size 3.2 1.6) (layers "F.Cu" "F.Mask") (roundrect_rratio 0.5) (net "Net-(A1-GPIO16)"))
  (pad "22" smd roundrect (at 9.69 21.59 270) (size 3.2 1.6) (layers "F.Cu" "F.Mask") (roundrect_rratio 0.5) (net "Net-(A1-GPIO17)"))
  (pad "23" smd custom (at 9.69 19.05 270) (size 1.6 0.8) (layers "F.Cu" "F.Mask") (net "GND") (options (clearance outline) (anchor rect))
   (primitives))
  (pad "24" smd roundrect (at 9.69 16.51 270) (size 3.2 1.6) (layers "F.Cu" "F.Mask") (roundrect_rratio 0.5)
   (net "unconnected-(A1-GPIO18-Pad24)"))
  (pad "25" smd roundrect (at 9.69 13.97 270) (size 3.2 1.6) (layers "F.Cu" "F.Mask") (roundrect_rratio 0.5) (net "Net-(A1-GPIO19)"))
  (pad "26" smd roundrect (at 9.69 11.43 270) (size 3.2 1.6) (layers "F.Cu" "F.Mask") (roundrect_rratio 0.5) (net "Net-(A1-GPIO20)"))
  (pad "27" smd roundrect (at 9.69 8.89 270) (size 3.2 1.6) (layers "F.Cu" "F.Mask") (roundrect_rratio 0.5) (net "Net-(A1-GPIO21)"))
  (pad "28" smd custom (at 9.69 6.35 270) (size 1.6 0.8) (layers "F.Cu" "F.Mask") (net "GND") (options (clearance outline) (anchor rect))
   (primitives))
  (pad "29" smd roundrect (at 9.69 3.81 270) (size 3.2 1.6) (layers "F.Cu" "F.Mask") (roundrect_rratio 0.5) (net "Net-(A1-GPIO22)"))
  (pad "30" smd roundrect (at 9.69 1.27 270) (size 3.2 1.6) (layers "F.Cu" "F.Mask") (roundrect_rratio 0.5)
   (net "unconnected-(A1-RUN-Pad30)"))
  (pad "31" smd roundrect (at 9.69 -1.27 270) (size 3.2 1.6) (layers "F.Cu" "F.Mask") (roundrect_rratio 0.5) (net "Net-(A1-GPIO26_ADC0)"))
  (pad "32" smd roundrect (at 9.69 -3.81 270) (size 3.2 1.6) (layers "F.Cu" "F.Mask") (roundrect_rratio 0.5) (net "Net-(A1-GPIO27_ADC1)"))
  (pad "33" smd custom (at 9.69 -6.35 270) (size 1.6 0.8) (layers "F.Cu" "F.Mask") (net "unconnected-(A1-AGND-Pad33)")
   (options (clearance outline) (anchor rect)) (primitives))
  (pad "34" smd roundrect (at 9.69 -8.89 270) (size 3.2 1.6) (layers "F.Cu" "F.Mask") (roundrect_rratio 0.5) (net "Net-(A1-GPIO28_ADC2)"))
  (pad "35" smd roundrect (at 9.69 -11.43 270) (size 3.2 1.6) (layers "F.Cu" "F.Mask") (roundrect_rratio 0.5)
   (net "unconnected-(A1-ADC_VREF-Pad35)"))
  (pad "36" smd roundrect (at 9.69 -13.97 270) (size 3.2 1.6) (layers "F.Cu" "F.Mask") (roundrect_rratio 0.5) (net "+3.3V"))
  (pad "37" smd roundrect (at 9.69 -16.51 270) (size 3.2 1.6) (layers "F.Cu" "F.Mask") (roundrect_rratio 0.5)
   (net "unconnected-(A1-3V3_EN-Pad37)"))
  (pad "38" smd custom (at 9.69 -19.05 270) (size 1.6 0.8) (layers "F.Cu" "F.Mask") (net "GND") (options (clearance outline) (anchor rect))
   (primitives))
  (pad "39" smd roundrect (at 9.69 -21.59 270) (size 3.2 1.6) (layers "F.Cu" "F.Mask") (roundrect_rratio 0.5) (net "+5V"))
  (pad "40" smd roundrect (at 9.69 -24.13 270) (size 3.2 1.6) (layers "F.Cu" "F.Mask") (roundrect_rratio 0.5)
   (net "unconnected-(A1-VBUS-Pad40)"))
  (pad "D1" smd roundrect (at -2.54 23.9) (size 3.2 1.6) (drill (offset -0.8 0)) (layers "F.Cu" "F.Mask") (roundrect_rratio 0.5)
   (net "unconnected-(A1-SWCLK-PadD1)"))
  (pad "D2" smd custom (at 0 23.9 180) (size 1.6 1.6) (layers "F.Cu" "F.Mask") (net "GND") (options (clearance outline) (anchor circle))
   (primitives))
  (pad "D3" smd roundrect (at 2.54 23.9) (size 3.2 1.6) (drill (offset -0.8 0)) (layers "F.Cu" "F.Mask") (roundrect_rratio 0.5)
   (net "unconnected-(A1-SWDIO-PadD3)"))
  (pad "TP1" smd roundrect (at 0 -21 270) (size 1.5 1.5) (layers "F.Cu" "F.Mask" "F.Paste") (roundrect_rratio 0.2)
   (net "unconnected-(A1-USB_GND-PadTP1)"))
  (pad "TP2" smd roundrect (at 1 -24.3 270) (size 1.5 1.5) (layers "F.Cu" "F.Mask" "F.Paste") (roundrect_rratio 0.2)
   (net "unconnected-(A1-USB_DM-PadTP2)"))
  (pad "TP3" smd roundrect (at -1 -24.3 270) (size 1.5 1.5) (layers "F.Cu" "F.Mask" "F.Paste") (roundrect_rratio 0.2)
   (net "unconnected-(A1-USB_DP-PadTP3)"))
  (pad "TP4" smd roundrect (at -2.5 -17.5 270) (size 1.5 1.5) (layers "F.Cu" "F.Mask" "F.Paste") (roundrect_rratio 0.2)
   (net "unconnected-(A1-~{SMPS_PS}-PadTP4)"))
  (pad "TP5" smd roundrect (at -2.5 -15 270) (size 1.5 1.5) (layers "F.Cu" "F.Mask" "F.Paste") (roundrect_rratio 0.2)
   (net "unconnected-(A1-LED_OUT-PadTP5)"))
  (pad "TP6" smd roundrect (at -2.5 -12.5 270) (size 1.5 1.5) (layers "F.Cu" "F.Mask" "F.Paste") (roundrect_rratio 0.2)
   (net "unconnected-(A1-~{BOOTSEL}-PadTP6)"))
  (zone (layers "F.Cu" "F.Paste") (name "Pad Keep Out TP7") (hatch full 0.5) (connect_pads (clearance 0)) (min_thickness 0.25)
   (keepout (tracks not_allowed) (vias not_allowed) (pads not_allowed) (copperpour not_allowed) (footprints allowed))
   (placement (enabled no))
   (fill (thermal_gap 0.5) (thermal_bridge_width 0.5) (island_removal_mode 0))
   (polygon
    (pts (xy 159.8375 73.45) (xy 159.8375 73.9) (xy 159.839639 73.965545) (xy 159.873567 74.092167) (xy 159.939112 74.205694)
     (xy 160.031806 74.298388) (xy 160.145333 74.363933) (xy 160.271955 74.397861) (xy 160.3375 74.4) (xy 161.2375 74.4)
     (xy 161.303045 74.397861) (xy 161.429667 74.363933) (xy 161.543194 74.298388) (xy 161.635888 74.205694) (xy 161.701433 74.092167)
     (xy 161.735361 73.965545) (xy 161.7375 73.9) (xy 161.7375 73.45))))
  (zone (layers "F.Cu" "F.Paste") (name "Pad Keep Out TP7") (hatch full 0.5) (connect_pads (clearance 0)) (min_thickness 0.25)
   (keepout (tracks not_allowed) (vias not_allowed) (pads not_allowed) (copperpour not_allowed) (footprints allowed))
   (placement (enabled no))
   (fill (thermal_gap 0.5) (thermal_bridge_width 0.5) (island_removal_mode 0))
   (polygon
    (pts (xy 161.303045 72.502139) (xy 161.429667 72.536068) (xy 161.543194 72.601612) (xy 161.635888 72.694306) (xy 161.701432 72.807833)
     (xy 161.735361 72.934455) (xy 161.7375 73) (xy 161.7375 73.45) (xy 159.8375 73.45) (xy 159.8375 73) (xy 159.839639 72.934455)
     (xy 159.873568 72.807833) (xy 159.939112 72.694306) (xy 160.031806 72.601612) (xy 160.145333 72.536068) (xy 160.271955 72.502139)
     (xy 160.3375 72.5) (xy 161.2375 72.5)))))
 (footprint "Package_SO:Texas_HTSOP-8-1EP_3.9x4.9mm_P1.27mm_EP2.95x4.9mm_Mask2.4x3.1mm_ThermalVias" (layer "F.Cu") (at 98.06 87.165 -90)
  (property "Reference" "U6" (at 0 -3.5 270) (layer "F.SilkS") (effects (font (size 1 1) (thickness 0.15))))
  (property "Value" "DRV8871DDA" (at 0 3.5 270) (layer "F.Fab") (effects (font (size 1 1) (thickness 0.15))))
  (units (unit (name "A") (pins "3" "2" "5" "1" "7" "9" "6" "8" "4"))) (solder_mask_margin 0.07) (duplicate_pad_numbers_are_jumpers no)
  (pad "" smd rect (at 0 0 270) (size 2.4 3.1) (layers "F.Mask"))
  (pad "" smd rect (at 0 0 270) (size 2.4 3.1) (layers "F.Paste"))
  (pad "1" smd rect (at -2.875 -1.905 270) (size 2.2 0.5) (layers "F.Cu" "F.Mask" "F.Paste") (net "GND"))
  (pad "2" smd rect (at -2.875 -0.635 270) (size 2.2 0.5) (layers "F.Cu" "F.Mask" "F.Paste") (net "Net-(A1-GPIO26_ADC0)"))
  (pad "3" smd rect (at -2.875 0.635 270) (size 2.2 0.5) (layers "F.Cu" "F.Mask" "F.Paste") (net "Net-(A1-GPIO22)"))
  (pad "4" smd rect (at -2.875 1.905 270) (size 2.2 0.5) (layers "F.Cu" "F.Mask" "F.Paste") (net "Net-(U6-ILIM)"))
  (pad "5" smd rect (at 2.875 1.905 270) (size 2.2 0.5) (layers "F.Cu" "F.Mask" "F.Paste") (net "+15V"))
  (pad "6" smd rect (at 2.875 0.635 270) (size 2.2 0.5) (layers "F.Cu" "F.Mask" "F.Paste") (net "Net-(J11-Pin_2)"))
  (pad "7" smd rect (at 2.875 -0.635 270) (size 2.2 0.5) (layers "F.Cu" "F.Mask" "F.Paste") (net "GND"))
  (pad "8" smd rect (at 2.875 -1.905 270) (size 2.2 0.5) (layers "F.Cu" "F.Mask" "F.Paste") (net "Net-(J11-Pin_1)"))
  (pad "9" thru_hole circle (at -0.65 -1.3 270) (size 0.63 0.63) (drill 0.33) (layers "*.Cu" "*.Mask") (remove_unused_layers no) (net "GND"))
  (pad "9" thru_hole circle (at -0.65 0 270) (size 0.63 0.63) (drill 0.33) (layers "*.Cu" "*.Mask") (remove_unused_layers no) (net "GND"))
  (pad "9" thru_hole circle (at -0.65 1.3 270) (size 0.63 0.63) (drill 0.33) (layers "*.Cu" "*.Mask") (remove_unused_layers no) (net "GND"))
  (pad "9" smd rect (at 0 0 270) (size 2.6 3.3) (layers "B.Cu") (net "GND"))
  (pad "9" smd rect (at 0 0 270) (size 2.95 4.9) (layers "F.Cu") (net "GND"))
  (pad "9" thru_hole circle (at 0.65 -1.3 270) (size 0.63 0.63) (drill 0.33) (layers "*.Cu" "*.Mask") (remove_unused_layers no) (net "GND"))
  (pad "9" thru_hole circle (at 0.65 0 270) (size 0.63 0.63) (drill 0.33) (layers "*.Cu" "*.Mask") (remove_unused_layers no) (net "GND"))
  (pad "9" thru_hole circle (at 0.65 1.3 270) (size 0.63 0.63) (drill 0.33) (layers "*.Cu" "*.Mask") (remove_unused_layers no) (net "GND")))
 (gr_rect (start 47 92) (end 183 131) (stroke (width 0.05) (type solid)) (fill no) (layer "Edge.Cuts"))
 (segment (start 103.685 70.91) (end 104.7 71.925) (width 0.254) (layer "F.Cu") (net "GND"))
 (segment (start 105.05 72.275) (end 105.05 74.3) (width 0.254) (layer "F.Cu") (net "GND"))
 (segment (start 105.05 74.3) (end 104.775 74.575) (width 0.254) (layer "F.Cu") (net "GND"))
 (segment (start 103.685 65.65) (end 103.685 70.91) (width 0.254) (layer "F.Cu") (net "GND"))
 (segment (start 104.7 71.925) (end 105.05 72.275) (width 0.254) (layer "F.Cu") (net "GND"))
 (segment (start 106.525 71.925) (end 106.525 70.7) (width 0.254) (layer "F.Cu") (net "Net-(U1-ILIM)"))
 (segment (start 106.525 70.7) (end 107.5 69.725) (width 0.254) (layer "F.Cu") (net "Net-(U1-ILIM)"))
 (segment (start 107.495 67.591) (end 107.5 67.596) (width 0.254) (layer "F.Cu") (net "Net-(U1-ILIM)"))
 (segment (start 107.495 65.65) (end 107.495 67.591) (width 0.254) (layer "F.Cu") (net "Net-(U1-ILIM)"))
 (segment (start 106.875 72.275) (end 106.875 74.3) (width 0.254) (layer "F.Cu") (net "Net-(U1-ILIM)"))
 (segment (start 106.525 71.925) (end 106.875 72.275) (width 0.254) (layer "F.Cu") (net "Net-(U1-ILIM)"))
 (segment (start 106.875 74.3) (end 106.6 74.575) (width 0.254) (layer "F.Cu") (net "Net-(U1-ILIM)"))
 (via (at 107.5 69.725) (size 0.6) (drill 0.3) (layers "F.Cu" "B.Cu") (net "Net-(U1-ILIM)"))
 (via (at 107.5 67.596) (size 0.6) (drill 0.3) (layers "F.Cu" "B.Cu") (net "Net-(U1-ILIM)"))
 (segment (start 107.5 67.596) (end 107.5 69.725) (width 0.254) (layer "B.Cu") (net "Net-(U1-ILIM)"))
 (segment (start 112.25 69) (end 104.96 69) (width 0.254) (layer "F.Cu") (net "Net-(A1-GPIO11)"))
 (segment (start 112.275 59.5) (end 112.275 68.975) (width 0.254) (layer "F.Cu") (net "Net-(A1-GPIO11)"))
 (segment (start 114.175 57.6) (end 112.275 59.5) (width 0.254) (layer "F.Cu") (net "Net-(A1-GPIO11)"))
 (segment (start 144.3575 62.76) (end 144.3575 58.6575) (width 0.254) (layer "F.Cu") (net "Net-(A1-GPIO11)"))
 (segment (start 104.95 69) (end 104.955 68.995) (width 0.2) (layer "F.Cu") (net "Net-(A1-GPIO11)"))
 (segment (start 112.275 68.975) (end 112.25 69) (width 0.254) (layer "F.Cu") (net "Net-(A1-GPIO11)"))
 (segment (start 104.955 68.995) (end 104.955 65.65) (width 0.2) (layer "F.Cu") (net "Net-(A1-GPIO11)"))
 (segment (start 143.3 57.6) (end 114.175 57.6) (width 0.254) (layer "F.Cu") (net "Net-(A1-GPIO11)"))
 (segment (start 104.96 69) (end 104.955 68.995) (width 0.254) (layer "F.Cu") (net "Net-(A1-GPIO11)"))
 (segment (start 144.3575 58.6575) (end 143.3 57.6) (width 0.254) (layer "F.Cu") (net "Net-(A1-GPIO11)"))
 (segment (start 108.95 68.975) (end 108.925 69) (width 0.254) (layer "B.Cu") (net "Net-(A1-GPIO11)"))
 (segment (start 111.225 68.15) (end 106.24 68.15) (width 0.254) (layer "F.Cu") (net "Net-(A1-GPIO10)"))
 (segment (start 106.225 68.165) (end 106.215 68.175) (width 0.2) (layer "F.Cu") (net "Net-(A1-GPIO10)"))
 (segment (start 106.225 65.65) (end 106.225 68.165) (width 0.2) (layer "F.Cu") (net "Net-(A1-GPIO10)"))
 (segment (start 146.8975 59.3725) (end 143.95 56.425) (width 0.254) (layer "F.Cu") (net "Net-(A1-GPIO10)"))
 (segment (start 113.75 56.425) (end 111.225 58.95) (width 0.254) (layer "F.Cu") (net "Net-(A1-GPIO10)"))
 (segment (start 111.225 58.95) (end 111.225 68.15) (width 0.254) (layer "F.Cu") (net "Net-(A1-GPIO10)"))
 (segment (start 143.95 56.425) (end 113.75 56.425) (width 0.254) (layer "F.Cu") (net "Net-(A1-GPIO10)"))
 (segment (start 146.8975 62.76) (end 146.8975 59.3725) (width 0.254) (layer "F.Cu") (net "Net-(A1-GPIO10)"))
 (segment (start 106.24 68.15) (end 106.225 68.165) (width 0.254) (layer "F.Cu") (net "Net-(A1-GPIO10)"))
 (segment (start 106.24 68.15) (end 106.215 68.175) (width 0.254) (layer "B.Cu") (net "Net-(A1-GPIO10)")))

